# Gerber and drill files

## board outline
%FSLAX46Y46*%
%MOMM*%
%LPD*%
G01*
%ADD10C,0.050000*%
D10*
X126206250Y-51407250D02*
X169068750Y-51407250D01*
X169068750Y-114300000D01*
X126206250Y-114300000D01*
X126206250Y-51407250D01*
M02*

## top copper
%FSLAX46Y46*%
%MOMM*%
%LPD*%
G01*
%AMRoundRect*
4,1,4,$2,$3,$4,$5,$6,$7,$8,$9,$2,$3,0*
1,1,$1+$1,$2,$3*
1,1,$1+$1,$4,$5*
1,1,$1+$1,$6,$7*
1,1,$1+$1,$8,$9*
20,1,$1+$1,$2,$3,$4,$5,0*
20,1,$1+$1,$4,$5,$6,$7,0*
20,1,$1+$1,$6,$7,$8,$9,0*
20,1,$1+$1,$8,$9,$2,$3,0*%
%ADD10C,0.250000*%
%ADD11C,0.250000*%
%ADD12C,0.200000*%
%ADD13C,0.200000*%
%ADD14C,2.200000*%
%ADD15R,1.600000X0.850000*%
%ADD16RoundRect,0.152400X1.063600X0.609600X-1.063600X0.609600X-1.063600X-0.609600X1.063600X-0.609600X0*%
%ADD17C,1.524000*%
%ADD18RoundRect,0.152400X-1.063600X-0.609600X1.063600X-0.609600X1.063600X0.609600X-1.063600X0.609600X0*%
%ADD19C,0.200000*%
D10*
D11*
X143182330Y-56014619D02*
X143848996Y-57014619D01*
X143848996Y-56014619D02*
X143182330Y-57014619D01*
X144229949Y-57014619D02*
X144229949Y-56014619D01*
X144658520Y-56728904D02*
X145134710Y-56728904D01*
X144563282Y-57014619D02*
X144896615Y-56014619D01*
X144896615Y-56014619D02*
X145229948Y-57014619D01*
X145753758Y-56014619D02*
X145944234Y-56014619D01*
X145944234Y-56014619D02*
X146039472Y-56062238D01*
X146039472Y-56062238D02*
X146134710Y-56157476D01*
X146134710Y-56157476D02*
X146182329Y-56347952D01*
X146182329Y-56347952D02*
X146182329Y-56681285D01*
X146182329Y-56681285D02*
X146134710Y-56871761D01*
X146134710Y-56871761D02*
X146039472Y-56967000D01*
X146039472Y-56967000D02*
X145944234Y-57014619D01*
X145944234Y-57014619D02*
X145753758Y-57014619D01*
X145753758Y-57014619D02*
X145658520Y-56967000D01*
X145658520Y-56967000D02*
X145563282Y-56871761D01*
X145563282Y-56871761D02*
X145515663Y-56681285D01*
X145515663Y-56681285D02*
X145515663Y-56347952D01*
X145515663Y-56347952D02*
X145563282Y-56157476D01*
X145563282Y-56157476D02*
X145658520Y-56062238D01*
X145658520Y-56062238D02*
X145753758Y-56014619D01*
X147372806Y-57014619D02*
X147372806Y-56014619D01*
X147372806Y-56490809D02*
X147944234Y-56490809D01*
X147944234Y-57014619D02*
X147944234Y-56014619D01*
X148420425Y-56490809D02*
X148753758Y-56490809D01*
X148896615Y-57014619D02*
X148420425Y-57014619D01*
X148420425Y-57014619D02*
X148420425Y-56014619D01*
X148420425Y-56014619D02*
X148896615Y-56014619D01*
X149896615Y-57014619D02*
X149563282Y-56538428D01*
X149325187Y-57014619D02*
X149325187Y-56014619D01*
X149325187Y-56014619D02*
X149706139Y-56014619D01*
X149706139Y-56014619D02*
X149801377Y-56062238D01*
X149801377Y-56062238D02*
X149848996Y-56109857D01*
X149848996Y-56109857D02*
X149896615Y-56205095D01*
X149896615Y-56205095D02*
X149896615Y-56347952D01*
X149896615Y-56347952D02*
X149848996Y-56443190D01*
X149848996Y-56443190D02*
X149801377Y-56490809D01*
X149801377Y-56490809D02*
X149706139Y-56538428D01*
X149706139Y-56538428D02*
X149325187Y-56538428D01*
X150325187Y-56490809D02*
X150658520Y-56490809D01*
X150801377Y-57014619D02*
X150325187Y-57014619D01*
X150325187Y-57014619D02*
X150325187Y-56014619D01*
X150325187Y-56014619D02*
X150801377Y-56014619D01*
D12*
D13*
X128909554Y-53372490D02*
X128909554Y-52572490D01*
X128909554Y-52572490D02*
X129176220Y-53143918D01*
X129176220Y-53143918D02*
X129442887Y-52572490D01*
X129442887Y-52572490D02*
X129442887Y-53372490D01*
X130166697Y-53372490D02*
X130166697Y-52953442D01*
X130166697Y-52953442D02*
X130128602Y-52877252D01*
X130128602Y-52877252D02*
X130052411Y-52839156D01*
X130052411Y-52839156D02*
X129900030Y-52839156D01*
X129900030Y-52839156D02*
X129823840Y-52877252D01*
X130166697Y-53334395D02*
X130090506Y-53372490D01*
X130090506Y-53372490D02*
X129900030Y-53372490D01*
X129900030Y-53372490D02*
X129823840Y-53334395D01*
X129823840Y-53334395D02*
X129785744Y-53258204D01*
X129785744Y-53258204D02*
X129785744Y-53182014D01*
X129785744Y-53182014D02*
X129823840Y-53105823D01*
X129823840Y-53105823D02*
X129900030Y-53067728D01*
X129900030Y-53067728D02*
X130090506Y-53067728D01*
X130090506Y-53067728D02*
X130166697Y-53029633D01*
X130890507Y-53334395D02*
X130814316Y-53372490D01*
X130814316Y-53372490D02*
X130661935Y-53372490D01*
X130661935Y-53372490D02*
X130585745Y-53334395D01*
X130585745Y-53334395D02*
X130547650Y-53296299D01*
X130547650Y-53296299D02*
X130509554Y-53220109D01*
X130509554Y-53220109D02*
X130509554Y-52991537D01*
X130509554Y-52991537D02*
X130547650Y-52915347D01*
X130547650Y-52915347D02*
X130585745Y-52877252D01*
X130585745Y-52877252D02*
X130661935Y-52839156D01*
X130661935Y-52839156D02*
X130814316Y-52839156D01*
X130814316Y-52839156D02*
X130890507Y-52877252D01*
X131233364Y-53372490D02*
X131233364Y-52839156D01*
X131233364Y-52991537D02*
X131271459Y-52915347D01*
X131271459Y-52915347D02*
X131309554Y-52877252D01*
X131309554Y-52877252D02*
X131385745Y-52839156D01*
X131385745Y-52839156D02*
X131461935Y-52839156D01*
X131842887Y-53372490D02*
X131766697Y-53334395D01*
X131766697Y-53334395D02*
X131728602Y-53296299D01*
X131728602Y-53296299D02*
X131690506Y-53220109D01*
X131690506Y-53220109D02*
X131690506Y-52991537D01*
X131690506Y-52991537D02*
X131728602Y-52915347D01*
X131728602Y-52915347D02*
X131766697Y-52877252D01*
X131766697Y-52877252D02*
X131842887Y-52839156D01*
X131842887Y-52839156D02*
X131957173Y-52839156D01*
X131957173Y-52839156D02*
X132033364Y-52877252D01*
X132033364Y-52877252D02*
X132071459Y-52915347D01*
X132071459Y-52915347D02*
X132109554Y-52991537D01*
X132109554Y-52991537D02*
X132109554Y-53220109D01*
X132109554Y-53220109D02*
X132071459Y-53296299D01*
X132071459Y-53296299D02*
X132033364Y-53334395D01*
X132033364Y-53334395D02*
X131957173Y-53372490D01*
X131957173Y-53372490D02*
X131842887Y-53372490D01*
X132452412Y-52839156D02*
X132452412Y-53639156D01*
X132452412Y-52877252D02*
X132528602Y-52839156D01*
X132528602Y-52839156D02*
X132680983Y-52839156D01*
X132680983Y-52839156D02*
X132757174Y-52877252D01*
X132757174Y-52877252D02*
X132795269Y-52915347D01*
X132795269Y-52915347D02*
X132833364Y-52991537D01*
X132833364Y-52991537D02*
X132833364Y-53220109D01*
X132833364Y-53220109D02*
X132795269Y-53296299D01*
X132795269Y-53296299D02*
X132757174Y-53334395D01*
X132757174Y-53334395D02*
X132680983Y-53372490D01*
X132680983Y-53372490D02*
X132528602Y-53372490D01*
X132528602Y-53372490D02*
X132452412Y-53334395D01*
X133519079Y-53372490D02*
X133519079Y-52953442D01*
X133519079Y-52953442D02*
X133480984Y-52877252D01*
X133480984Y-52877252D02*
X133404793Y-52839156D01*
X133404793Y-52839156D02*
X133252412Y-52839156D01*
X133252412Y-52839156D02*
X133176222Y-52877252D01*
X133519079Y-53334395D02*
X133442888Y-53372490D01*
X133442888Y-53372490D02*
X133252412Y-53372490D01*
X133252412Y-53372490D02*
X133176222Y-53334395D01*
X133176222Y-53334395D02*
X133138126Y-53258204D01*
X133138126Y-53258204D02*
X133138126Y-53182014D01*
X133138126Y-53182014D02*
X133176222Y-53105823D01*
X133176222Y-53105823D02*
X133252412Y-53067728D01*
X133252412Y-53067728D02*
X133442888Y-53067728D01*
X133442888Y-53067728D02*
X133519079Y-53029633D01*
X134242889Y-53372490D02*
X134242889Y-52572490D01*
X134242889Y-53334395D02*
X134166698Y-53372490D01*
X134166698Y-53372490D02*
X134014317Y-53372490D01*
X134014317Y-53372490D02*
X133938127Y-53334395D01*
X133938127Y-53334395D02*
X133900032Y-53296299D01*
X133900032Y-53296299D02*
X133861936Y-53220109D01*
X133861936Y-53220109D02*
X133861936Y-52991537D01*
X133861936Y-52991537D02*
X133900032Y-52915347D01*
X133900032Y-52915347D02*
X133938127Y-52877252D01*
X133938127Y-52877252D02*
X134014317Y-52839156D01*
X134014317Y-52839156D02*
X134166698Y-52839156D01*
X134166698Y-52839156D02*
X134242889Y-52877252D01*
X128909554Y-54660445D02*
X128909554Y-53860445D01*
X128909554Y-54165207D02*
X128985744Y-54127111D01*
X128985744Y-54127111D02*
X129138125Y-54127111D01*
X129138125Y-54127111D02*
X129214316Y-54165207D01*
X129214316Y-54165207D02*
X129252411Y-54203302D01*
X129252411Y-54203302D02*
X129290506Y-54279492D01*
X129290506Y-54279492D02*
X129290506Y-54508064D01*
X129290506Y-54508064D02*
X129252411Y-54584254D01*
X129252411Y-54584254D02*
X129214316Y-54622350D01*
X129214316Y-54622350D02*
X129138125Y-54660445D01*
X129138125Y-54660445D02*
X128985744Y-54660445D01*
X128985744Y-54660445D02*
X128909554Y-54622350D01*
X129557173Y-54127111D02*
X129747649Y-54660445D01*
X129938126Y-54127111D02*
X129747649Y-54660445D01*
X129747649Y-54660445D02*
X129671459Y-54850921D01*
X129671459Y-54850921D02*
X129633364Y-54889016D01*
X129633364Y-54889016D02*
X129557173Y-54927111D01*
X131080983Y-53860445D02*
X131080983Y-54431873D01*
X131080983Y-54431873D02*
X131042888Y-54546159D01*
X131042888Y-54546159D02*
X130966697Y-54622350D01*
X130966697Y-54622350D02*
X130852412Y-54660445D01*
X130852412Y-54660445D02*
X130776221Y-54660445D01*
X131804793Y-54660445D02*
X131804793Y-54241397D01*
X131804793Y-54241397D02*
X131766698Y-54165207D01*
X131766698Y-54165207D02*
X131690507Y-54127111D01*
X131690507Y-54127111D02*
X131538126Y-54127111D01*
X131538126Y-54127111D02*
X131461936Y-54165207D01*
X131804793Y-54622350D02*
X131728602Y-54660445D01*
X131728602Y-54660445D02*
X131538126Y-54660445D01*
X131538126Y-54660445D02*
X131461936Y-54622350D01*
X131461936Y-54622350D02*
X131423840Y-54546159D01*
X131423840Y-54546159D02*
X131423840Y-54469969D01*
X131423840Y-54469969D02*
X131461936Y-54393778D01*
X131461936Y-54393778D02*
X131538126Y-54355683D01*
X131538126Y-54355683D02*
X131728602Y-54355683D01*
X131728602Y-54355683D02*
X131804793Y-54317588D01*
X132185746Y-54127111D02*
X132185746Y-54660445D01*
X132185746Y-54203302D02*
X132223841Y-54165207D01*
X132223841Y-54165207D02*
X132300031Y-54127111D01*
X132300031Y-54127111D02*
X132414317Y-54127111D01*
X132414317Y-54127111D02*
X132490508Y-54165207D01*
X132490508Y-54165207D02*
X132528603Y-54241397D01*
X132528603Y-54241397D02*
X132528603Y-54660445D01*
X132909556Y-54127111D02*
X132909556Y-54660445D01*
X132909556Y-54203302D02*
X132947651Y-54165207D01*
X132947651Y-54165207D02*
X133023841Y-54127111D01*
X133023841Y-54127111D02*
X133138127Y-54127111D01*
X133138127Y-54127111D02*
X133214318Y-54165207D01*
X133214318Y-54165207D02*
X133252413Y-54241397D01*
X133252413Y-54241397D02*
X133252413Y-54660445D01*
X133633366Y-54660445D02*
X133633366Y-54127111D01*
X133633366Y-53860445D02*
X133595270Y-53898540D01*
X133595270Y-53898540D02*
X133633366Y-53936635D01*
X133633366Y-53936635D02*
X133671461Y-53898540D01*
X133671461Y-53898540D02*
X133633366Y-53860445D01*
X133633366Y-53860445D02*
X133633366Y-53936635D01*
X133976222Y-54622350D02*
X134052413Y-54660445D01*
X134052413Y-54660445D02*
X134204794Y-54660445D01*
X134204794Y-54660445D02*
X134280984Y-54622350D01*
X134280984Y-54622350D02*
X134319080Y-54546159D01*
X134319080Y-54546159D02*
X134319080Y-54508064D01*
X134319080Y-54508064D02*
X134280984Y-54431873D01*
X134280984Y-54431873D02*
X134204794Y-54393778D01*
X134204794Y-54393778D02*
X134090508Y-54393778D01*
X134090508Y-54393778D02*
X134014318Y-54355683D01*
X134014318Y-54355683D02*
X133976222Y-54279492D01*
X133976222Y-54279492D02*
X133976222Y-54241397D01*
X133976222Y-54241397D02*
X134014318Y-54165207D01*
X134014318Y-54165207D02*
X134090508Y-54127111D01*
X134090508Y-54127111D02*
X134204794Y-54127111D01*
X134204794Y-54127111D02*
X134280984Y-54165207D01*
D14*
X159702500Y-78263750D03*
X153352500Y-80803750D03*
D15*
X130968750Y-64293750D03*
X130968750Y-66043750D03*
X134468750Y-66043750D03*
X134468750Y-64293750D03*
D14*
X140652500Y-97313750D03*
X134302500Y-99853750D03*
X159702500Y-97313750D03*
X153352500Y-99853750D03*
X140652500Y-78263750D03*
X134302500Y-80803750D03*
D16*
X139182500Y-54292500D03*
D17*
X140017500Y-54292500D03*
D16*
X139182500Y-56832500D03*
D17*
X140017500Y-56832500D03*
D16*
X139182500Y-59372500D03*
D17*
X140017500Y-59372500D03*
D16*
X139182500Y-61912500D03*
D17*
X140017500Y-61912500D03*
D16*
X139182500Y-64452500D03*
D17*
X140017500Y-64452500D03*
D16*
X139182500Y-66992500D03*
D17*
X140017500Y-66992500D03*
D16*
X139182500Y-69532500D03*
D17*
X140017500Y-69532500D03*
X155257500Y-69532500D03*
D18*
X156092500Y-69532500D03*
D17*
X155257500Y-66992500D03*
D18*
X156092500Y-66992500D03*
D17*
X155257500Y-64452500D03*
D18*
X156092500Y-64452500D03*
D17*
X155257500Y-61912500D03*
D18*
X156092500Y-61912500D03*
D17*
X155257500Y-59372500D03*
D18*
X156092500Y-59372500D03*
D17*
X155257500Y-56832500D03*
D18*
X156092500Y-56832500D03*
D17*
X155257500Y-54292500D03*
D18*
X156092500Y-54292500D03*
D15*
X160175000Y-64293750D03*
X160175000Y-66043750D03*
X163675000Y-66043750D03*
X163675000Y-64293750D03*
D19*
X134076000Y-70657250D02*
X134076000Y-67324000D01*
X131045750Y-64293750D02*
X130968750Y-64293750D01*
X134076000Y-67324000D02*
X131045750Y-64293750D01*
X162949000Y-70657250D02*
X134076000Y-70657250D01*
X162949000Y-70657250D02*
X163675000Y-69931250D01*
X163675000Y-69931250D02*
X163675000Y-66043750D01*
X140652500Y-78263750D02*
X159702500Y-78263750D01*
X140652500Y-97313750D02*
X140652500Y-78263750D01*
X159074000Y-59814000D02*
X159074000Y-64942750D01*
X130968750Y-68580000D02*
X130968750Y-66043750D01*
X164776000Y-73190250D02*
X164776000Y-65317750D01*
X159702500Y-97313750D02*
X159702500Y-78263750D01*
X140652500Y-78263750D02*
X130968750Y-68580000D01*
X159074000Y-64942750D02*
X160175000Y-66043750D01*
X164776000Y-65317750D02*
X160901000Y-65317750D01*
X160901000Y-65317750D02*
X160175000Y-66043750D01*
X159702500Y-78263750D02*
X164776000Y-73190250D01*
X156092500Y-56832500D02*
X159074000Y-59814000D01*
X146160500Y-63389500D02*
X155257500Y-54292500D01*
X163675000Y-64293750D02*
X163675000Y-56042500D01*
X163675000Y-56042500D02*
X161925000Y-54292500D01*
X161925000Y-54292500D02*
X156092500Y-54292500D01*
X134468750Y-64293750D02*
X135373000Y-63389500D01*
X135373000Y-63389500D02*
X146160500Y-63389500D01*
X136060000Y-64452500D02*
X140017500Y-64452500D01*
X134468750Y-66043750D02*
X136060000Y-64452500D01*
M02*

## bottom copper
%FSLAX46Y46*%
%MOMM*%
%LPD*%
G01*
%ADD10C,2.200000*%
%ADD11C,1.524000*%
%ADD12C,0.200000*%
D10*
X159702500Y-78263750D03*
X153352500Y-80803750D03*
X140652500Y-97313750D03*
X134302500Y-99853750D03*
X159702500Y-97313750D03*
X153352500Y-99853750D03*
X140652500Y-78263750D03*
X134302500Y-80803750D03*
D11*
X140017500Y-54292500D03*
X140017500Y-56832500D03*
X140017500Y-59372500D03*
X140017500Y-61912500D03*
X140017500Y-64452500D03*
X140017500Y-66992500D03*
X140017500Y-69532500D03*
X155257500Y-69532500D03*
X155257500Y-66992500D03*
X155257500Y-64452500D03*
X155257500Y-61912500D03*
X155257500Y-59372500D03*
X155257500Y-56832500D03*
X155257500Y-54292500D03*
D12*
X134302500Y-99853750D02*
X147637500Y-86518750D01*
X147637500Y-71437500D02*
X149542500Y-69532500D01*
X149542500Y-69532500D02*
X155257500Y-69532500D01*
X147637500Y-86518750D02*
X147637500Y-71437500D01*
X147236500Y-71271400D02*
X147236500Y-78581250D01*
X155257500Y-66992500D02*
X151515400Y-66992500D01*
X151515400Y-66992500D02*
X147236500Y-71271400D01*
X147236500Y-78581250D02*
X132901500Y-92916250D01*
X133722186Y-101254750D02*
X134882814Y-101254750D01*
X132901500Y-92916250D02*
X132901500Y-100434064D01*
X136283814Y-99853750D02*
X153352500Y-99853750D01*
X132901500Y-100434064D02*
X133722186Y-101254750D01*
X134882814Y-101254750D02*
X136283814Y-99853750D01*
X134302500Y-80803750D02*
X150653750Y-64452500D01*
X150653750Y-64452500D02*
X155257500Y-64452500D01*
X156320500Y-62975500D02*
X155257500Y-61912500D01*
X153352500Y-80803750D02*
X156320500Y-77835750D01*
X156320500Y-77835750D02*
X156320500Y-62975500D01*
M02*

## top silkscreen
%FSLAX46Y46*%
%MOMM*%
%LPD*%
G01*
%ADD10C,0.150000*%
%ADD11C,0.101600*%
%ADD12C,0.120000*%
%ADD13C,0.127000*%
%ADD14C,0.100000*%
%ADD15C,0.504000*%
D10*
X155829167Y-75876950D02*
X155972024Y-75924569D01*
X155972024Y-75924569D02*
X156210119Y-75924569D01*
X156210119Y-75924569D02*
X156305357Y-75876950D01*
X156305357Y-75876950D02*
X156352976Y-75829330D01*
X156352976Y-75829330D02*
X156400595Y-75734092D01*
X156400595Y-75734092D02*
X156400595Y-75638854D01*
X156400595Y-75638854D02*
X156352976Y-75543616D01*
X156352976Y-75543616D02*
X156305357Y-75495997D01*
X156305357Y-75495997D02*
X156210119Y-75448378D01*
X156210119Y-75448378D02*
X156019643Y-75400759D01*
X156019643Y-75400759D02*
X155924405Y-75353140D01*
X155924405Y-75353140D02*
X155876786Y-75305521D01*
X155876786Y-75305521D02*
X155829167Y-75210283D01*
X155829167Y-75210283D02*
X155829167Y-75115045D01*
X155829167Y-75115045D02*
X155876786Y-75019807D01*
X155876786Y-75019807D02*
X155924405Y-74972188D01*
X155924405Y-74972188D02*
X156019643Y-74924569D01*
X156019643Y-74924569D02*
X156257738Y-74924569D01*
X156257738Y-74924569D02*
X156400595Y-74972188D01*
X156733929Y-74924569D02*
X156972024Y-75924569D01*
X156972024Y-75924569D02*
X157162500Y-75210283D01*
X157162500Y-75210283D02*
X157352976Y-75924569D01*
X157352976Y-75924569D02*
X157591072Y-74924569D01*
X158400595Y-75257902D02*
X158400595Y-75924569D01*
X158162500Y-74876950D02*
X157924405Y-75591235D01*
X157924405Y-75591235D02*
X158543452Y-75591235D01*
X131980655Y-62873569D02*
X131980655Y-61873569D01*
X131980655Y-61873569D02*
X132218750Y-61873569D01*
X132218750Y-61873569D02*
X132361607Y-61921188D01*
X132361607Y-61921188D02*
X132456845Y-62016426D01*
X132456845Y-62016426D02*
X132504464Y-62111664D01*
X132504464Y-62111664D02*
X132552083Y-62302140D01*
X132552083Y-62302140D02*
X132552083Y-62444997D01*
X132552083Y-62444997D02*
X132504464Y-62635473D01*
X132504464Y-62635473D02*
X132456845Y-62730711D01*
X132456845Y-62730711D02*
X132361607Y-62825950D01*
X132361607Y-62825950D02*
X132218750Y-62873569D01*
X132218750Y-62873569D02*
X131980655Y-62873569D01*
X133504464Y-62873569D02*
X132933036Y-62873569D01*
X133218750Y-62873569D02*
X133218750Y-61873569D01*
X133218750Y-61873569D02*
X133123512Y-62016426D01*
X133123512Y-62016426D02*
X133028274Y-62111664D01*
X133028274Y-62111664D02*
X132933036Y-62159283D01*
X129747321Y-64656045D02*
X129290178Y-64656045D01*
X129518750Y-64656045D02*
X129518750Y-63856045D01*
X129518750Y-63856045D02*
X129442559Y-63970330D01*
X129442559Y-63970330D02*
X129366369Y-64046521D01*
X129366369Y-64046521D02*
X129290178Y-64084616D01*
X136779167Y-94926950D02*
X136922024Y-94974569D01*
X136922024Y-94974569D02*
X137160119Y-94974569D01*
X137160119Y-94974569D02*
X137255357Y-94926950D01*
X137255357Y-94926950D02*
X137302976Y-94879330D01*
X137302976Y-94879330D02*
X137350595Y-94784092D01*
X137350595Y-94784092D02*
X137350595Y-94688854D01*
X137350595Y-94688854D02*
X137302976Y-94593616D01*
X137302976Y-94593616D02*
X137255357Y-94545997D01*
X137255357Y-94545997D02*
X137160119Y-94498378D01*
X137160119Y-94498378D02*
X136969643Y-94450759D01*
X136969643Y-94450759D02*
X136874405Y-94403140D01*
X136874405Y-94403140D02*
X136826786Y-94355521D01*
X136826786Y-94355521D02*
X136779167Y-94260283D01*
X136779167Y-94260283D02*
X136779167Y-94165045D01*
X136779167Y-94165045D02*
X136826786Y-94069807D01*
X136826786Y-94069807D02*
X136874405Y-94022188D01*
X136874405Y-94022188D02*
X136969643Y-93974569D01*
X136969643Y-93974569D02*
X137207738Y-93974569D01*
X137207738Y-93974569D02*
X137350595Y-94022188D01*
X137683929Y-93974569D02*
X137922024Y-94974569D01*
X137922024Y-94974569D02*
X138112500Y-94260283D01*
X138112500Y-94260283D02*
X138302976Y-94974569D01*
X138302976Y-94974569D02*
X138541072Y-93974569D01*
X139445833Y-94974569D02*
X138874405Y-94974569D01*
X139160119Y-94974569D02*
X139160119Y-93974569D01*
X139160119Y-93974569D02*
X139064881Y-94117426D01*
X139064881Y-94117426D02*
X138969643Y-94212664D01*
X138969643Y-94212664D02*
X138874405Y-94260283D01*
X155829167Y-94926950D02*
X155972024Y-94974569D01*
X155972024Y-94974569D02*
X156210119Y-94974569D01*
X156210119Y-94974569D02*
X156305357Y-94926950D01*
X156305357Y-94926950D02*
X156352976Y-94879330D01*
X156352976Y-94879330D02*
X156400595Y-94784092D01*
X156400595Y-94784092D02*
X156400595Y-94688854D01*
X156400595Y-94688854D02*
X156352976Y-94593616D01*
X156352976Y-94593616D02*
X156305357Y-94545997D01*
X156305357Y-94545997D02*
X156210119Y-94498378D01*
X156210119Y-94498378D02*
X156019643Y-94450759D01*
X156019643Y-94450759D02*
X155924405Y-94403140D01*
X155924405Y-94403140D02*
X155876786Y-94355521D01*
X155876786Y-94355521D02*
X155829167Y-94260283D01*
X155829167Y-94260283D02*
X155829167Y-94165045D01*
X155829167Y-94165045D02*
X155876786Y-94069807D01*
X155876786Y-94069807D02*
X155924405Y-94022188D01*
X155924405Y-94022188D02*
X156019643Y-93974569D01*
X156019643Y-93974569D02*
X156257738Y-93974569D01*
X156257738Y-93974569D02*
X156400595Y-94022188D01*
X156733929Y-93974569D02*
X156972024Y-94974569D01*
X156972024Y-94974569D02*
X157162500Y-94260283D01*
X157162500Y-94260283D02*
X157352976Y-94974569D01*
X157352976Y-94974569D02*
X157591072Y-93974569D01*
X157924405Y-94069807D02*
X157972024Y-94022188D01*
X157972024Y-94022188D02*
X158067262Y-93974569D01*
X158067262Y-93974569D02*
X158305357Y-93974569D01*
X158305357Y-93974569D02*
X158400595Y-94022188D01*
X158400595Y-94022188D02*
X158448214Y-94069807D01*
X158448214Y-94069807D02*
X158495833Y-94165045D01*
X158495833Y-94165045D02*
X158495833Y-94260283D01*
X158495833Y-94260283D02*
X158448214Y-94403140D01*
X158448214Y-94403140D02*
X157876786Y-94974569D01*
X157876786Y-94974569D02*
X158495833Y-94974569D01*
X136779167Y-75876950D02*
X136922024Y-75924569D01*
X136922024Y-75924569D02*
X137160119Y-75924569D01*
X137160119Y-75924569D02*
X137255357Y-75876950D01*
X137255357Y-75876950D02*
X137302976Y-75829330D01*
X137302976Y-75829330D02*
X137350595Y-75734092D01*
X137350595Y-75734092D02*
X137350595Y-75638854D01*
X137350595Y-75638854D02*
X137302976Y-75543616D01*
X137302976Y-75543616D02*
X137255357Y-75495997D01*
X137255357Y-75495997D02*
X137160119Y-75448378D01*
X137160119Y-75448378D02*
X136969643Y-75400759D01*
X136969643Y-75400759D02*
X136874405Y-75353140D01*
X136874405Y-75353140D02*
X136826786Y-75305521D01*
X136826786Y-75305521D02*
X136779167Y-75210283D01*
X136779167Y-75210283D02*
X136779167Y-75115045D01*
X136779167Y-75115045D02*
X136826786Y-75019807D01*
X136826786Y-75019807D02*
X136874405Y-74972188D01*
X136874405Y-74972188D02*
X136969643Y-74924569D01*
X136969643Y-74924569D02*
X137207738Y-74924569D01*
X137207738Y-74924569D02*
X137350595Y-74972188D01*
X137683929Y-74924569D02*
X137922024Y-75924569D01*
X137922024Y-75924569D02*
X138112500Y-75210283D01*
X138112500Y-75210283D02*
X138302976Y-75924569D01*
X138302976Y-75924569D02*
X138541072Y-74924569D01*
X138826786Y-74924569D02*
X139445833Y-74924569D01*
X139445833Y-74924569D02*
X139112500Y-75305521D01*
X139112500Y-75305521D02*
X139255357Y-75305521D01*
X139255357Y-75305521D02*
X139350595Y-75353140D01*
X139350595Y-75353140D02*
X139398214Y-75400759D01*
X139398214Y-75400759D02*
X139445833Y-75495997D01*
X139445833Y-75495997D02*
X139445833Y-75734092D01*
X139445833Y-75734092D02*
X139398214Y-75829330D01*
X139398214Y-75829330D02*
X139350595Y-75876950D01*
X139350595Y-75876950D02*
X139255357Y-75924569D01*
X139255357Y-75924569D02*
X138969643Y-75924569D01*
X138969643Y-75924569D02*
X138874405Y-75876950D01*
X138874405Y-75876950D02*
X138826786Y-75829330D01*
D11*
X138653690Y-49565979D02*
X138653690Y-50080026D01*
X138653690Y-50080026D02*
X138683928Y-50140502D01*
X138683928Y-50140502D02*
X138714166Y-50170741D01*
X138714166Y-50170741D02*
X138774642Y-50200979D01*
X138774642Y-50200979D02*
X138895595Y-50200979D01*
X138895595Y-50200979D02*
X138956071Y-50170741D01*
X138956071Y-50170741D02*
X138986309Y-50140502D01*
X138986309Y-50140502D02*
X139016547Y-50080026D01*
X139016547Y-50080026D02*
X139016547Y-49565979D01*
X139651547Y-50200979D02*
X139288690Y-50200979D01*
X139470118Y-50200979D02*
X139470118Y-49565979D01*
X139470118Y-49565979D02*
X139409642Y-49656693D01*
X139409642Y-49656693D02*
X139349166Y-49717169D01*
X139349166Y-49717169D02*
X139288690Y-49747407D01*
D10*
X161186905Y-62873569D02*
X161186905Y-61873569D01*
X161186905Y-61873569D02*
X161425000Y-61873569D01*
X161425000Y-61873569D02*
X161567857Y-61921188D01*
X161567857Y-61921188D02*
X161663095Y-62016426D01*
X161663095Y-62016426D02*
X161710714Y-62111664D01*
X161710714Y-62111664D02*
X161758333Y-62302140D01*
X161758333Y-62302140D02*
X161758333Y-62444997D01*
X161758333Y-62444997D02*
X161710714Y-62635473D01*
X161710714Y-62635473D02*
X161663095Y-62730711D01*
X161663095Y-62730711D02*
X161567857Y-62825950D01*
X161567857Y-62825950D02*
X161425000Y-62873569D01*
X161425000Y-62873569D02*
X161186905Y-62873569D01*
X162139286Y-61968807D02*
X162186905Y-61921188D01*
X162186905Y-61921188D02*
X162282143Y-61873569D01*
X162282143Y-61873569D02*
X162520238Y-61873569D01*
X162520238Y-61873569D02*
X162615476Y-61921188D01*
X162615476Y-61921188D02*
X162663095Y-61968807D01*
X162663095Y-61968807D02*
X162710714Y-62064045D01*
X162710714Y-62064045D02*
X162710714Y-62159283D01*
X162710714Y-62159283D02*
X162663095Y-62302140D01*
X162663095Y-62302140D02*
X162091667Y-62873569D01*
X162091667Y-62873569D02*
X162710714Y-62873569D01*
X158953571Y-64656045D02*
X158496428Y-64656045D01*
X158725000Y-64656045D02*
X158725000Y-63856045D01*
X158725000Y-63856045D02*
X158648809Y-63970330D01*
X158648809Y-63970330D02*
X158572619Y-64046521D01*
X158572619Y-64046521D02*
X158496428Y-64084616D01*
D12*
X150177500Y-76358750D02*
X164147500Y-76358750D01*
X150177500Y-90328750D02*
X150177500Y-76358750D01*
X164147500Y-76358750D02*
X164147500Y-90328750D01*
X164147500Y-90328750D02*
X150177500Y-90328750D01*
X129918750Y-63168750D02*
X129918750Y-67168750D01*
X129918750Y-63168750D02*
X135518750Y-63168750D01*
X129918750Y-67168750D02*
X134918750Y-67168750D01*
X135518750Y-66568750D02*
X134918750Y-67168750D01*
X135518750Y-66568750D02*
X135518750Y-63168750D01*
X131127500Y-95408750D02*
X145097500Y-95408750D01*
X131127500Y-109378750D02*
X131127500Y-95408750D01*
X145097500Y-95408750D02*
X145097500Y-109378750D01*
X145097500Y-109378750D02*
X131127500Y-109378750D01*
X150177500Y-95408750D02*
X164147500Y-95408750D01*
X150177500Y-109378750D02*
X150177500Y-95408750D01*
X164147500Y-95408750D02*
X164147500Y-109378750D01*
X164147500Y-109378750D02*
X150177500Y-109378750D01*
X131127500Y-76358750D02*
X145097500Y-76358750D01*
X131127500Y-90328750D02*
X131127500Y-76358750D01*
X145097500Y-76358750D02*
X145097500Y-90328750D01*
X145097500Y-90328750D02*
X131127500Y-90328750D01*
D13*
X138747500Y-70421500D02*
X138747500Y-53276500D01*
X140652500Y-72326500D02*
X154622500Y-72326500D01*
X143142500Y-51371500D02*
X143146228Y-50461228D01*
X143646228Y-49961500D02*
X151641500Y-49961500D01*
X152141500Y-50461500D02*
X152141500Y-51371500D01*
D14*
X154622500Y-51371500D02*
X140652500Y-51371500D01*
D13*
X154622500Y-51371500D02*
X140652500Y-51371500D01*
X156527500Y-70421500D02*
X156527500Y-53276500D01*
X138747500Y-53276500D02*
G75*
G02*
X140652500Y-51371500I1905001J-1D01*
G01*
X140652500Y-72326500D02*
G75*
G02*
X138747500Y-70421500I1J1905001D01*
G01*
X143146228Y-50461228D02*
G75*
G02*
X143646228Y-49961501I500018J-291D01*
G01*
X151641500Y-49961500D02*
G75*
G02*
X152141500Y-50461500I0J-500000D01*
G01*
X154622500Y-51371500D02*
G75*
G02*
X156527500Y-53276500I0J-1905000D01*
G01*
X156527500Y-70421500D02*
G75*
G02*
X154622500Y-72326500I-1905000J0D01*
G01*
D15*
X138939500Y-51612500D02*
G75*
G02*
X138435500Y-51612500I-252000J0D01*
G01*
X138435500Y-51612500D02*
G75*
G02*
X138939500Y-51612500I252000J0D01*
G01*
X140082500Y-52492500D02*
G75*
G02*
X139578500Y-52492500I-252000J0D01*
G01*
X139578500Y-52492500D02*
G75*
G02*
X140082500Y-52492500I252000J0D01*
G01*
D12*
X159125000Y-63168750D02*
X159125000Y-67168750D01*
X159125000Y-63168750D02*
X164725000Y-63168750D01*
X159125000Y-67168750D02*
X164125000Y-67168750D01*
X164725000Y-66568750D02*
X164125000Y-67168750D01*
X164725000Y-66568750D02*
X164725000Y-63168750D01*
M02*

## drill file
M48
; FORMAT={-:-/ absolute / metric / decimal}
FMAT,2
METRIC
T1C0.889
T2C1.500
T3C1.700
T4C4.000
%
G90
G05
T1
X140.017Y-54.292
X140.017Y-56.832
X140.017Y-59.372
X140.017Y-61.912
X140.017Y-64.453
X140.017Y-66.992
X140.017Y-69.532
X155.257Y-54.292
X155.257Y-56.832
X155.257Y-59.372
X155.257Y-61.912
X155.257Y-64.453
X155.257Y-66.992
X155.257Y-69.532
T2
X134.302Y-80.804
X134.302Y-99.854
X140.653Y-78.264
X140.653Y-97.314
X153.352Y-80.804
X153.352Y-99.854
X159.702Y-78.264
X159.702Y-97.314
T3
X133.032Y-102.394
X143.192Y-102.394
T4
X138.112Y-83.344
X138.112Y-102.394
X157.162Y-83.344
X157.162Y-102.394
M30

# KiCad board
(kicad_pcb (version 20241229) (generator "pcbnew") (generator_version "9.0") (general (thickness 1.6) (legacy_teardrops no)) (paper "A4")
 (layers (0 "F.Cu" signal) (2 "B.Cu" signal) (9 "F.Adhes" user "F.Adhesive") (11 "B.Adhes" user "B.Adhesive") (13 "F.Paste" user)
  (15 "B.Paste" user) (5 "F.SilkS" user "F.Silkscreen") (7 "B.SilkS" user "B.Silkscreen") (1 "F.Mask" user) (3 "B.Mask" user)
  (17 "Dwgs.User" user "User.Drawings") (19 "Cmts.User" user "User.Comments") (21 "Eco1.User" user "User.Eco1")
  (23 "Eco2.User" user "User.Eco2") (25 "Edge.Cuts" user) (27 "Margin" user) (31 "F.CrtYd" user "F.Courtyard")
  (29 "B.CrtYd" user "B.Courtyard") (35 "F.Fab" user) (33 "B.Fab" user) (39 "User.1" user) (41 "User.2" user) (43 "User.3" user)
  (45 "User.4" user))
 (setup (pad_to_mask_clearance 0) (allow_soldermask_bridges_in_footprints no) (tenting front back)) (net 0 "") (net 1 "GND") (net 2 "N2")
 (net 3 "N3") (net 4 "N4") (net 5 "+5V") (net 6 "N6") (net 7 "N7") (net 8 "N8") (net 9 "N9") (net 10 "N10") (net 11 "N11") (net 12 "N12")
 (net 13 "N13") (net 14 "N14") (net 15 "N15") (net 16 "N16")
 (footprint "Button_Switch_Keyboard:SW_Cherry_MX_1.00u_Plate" (layer "F.Cu") (at 159.7025 78.26375)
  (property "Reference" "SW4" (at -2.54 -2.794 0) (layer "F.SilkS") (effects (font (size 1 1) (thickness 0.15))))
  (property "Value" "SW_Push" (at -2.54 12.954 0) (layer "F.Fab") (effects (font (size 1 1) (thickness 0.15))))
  (fp_line (start -9.525 -1.905) (end 4.445 -1.905) (stroke (width 0.12) (type solid)) (layer "F.SilkS"))
  (fp_line (start -9.525 12.065) (end -9.525 -1.905) (stroke (width 0.12) (type solid)) (layer "F.SilkS"))
  (fp_line (start 4.445 -1.905) (end 4.445 12.065) (stroke (width 0.12) (type solid)) (layer "F.SilkS"))
  (fp_line (start 4.445 12.065) (end -9.525 12.065) (stroke (width 0.12) (type solid)) (layer "F.SilkS"))
  (pad "" np_thru_hole circle (at -2.54 5.08) (size 4 4) (drill 4) (layers "*.Cu" "*.Mask"))
  (pad "1" thru_hole circle (at 0 0) (size 2.2 2.2) (drill 1.5) (layers "*.Cu" "*.Mask") (remove_unused_layers no) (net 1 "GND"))
  (pad "2" thru_hole circle (at -6.35 2.54) (size 2.2 2.2) (drill 1.5) (layers "*.Cu" "*.Mask") (remove_unused_layers no) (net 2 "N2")))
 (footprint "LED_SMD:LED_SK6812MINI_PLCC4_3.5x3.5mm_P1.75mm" (layer "F.Cu") (at 132.71875 65.16875)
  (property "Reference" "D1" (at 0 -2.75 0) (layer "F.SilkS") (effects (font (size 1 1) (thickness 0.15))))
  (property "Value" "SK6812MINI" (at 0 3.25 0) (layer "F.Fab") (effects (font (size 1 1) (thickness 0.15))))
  (fp_line (start -2.8 -2) (end -2.8 2) (stroke (width 0.12) (type default)) (layer "F.SilkS"))
  (fp_line (start -2.8 -2) (end 2.8 -2) (stroke (width 0.12) (type solid)) (layer "F.SilkS"))
  (fp_line (start -2.8 2) (end 2.2 2) (stroke (width 0.12) (type solid)) (layer "F.SilkS"))
  (fp_line (start 2.8 1.4) (end 2.2 2) (stroke (width 0.12) (type default)) (layer "F.SilkS"))
  (fp_line (start 2.8 1.4) (end 2.8 -2) (stroke (width 0.12) (type solid)) (layer "F.SilkS"))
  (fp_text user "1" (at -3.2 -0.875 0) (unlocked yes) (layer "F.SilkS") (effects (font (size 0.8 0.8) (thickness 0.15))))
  (pad "1" smd rect (at -1.75 -0.875) (size 1.6 0.85) (layers "F.Cu" "F.Mask" "F.Paste") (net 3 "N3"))
  (pad "2" smd rect (at -1.75 0.875) (size 1.6 0.85) (layers "F.Cu" "F.Mask" "F.Paste") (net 1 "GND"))
  (pad "3" smd rect (at 1.75 0.875) (size 1.6 0.85) (layers "F.Cu" "F.Mask" "F.Paste") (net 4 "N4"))
  (pad "4" smd rect (at 1.75 -0.875) (size 1.6 0.85) (layers "F.Cu" "F.Mask" "F.Paste") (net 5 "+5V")))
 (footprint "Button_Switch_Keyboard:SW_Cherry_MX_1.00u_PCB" (layer "F.Cu") (at 140.6525 97.31375)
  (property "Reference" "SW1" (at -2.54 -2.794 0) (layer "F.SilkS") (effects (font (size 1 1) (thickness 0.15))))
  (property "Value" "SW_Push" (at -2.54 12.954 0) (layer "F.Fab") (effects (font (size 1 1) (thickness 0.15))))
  (fp_line (start -9.525 -1.905) (end 4.445 -1.905) (stroke (width 0.12) (type solid)) (layer "F.SilkS"))
  (fp_line (start -9.525 12.065) (end -9.525 -1.905) (stroke (width 0.12) (type solid)) (layer "F.SilkS"))
  (fp_line (start 4.445 -1.905) (end 4.445 12.065) (stroke (width 0.12) (type solid)) (layer "F.SilkS"))
  (fp_line (start 4.445 12.065) (end -9.525 12.065) (stroke (width 0.12) (type solid)) (layer "F.SilkS"))
  (pad "" np_thru_hole circle (at -7.62 5.08) (size 1.7 1.7) (drill 1.7) (layers "*.Cu" "*.Mask"))
  (pad "" np_thru_hole circle (at -2.54 5.08) (size 4 4) (drill 4) (layers "*.Cu" "*.Mask"))
  (pad "" np_thru_hole circle (at 2.54 5.08) (size 1.7 1.7) (drill 1.7) (layers "*.Cu" "*.Mask"))
  (pad "1" thru_hole circle (at 0 0) (size 2.2 2.2) (drill 1.5) (layers "*.Cu" "*.Mask") (remove_unused_layers no) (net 1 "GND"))
  (pad "2" thru_hole circle (at -6.35 2.54) (size 2.2 2.2) (drill 1.5) (layers "*.Cu" "*.Mask") (remove_unused_layers no) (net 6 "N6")))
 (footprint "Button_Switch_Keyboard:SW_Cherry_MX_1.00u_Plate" (layer "F.Cu") (at 159.7025 97.31375)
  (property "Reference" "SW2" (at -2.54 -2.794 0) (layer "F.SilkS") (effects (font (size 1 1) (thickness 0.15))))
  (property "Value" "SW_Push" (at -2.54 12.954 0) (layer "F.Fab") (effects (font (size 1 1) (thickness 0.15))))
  (fp_line (start -9.525 -1.905) (end 4.445 -1.905) (stroke (width 0.12) (type solid)) (layer "F.SilkS"))
  (fp_line (start -9.525 12.065) (end -9.525 -1.905) (stroke (width 0.12) (type solid)) (layer "F.SilkS"))
  (fp_line (start 4.445 -1.905) (end 4.445 12.065) (stroke (width 0.12) (type solid)) (layer "F.SilkS"))
  (fp_line (start 4.445 12.065) (end -9.525 12.065) (stroke (width 0.12) (type solid)) (layer "F.SilkS"))
  (pad "" np_thru_hole circle (at -2.54 5.08) (size 4 4) (drill 4) (layers "*.Cu" "*.Mask"))
  (pad "1" thru_hole circle (at 0 0) (size 2.2 2.2) (drill 1.5) (layers "*.Cu" "*.Mask") (remove_unused_layers no) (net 1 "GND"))
  (pad "2" thru_hole circle (at -6.35 2.54) (size 2.2 2.2) (drill 1.5) (layers "*.Cu" "*.Mask") (remove_unused_layers no) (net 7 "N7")))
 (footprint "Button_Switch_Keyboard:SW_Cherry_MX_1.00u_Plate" (layer "F.Cu") (at 140.6525 78.26375)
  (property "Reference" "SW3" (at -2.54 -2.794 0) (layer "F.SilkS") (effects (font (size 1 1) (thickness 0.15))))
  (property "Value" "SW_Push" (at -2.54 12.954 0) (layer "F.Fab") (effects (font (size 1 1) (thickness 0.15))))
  (fp_line (start -9.525 -1.905) (end 4.445 -1.905) (stroke (width 0.12) (type solid)) (layer "F.SilkS"))
  (fp_line (start -9.525 12.065) (end -9.525 -1.905) (stroke (width 0.12) (type solid)) (layer "F.SilkS"))
  (fp_line (start 4.445 -1.905) (end 4.445 12.065) (stroke (width 0.12) (type solid)) (layer "F.SilkS"))
  (fp_line (start 4.445 12.065) (end -9.525 12.065) (stroke (width 0.12) (type solid)) (layer "F.SilkS"))
  (pad "" np_thru_hole circle (at -2.54 5.08) (size 4 4) (drill 4) (layers "*.Cu" "*.Mask"))
  (pad "1" thru_hole circle (at 0 0) (size 2.2 2.2) (drill 1.5) (layers "*.Cu" "*.Mask") (remove_unused_layers no) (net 1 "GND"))
  (pad "2" thru_hole circle (at -6.35 2.54) (size 2.2 2.2) (drill 1.5) (layers "*.Cu" "*.Mask") (remove_unused_layers no) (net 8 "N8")))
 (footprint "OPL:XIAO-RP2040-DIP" (layer "F.Cu") (at 147.6375 61.9125)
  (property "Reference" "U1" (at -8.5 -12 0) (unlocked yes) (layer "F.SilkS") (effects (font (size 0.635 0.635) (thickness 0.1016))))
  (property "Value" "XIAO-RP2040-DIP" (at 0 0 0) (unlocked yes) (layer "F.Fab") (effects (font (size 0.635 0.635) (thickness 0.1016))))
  (fp_line (start -8.89 8.509) (end -8.89 -8.636) (stroke (width 0.127) (type solid)) (layer "F.SilkS"))
  (fp_line (start -6.985 10.414) (end 6.985 10.414) (stroke (width 0.127) (type solid)) (layer "F.SilkS"))
  (fp_line (start -4.495 -10.541) (end -4.491272 -11.451272) (stroke (width 0.127) (type solid)) (layer "F.SilkS"))
  (fp_line (start -3.991272 -11.951) (end 4.004 -11.951) (stroke (width 0.127) (type solid)) (layer "F.SilkS"))
  (fp_line (start 4.504 -11.451) (end 4.504 -10.541) (stroke (width 0.127) (type solid)) (layer "F.SilkS"))
  (fp_line (start 6.985 -10.541) (end -6.985 -10.541) (stroke (width 0.1) (type solid)) (layer "F.SilkS"))
  (fp_line (start 6.985 -10.541) (end -6.985 -10.541) (stroke (width 0.127) (type solid)) (layer "F.SilkS"))
  (fp_line (start 8.89 8.509) (end 8.89 -8.636) (stroke (width 0.127) (type solid)) (layer "F.SilkS"))
  (fp_arc (start -8.89 -8.636) (mid -8.332038 -9.983038) (end -6.985 -10.541) (stroke (width 0.127) (type solid)) (layer "F.SilkS"))
  (fp_arc (start -6.985 10.414) (mid -8.332038 9.856038) (end -8.89 8.509) (stroke (width 0.127) (type solid)) (layer "F.SilkS"))
  (fp_arc (start -4.491272 -11.451272) (mid -4.344728 -11.80464) (end -3.991272 -11.951) (stroke (width 0.127) (type default))
   (layer "F.SilkS"))
  (fp_arc (start 4.004 -11.951) (mid 4.357553 -11.804553) (end 4.504 -11.451) (stroke (width 0.127) (type default)) (layer "F.SilkS"))
  (fp_arc (start 6.985 -10.541) (mid 8.332038 -9.983038) (end 8.89 -8.636) (stroke (width 0.127) (type solid)) (layer "F.SilkS"))
  (fp_arc (start 8.89 8.509) (mid 8.332038 9.856038) (end 6.985 10.414) (stroke (width 0.127) (type solid)) (layer "F.SilkS"))
  (fp_circle (center -8.95 -10.3) (end -8.95 -10.554) (stroke (width 0.5) (type solid)) (fill yes) (layer "F.SilkS"))
  (fp_circle (center -7.807 -9.42) (end -7.807 -9.674) (stroke (width 0.5) (type solid)) (fill yes) (layer "F.SilkS"))
  (pad "1" smd roundrect (at -8.455 -7.62 180) (size 2.432 1.524) (layers "F.Cu" "F.Mask") (roundrect_rratio 0.1) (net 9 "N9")
   (thermal_bridge_angle 45))
  (pad "1" thru_hole circle (at -7.62 -7.62 180) (size 1.524 1.524) (drill 0.889) (layers "*.Cu" "*.Mask") (remove_unused_layers no)
   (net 9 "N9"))
  (pad "2" smd roundrect (at -8.455 -5.08 180) (size 2.432 1.524) (layers "F.Cu" "F.Mask") (roundrect_rratio 0.1) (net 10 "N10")
   (thermal_bridge_angle 45))
  (pad "2" thru_hole circle (at -7.62 -5.08 180) (size 1.524 1.524) (drill 0.889) (layers "*.Cu" "*.Mask") (remove_unused_layers no)
   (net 10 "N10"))
  (pad "3" smd roundrect (at -8.455 -2.54 180) (size 2.432 1.524) (layers "F.Cu" "F.Mask") (roundrect_rratio 0.1) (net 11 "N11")
   (thermal_bridge_angle 45))
  (pad "3" thru_hole circle (at -7.62 -2.54 180) (size 1.524 1.524) (drill 0.889) (layers "*.Cu" "*.Mask") (remove_unused_layers no)
   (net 11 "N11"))
  (pad "4" smd roundrect (at -8.455 0 180) (size 2.432 1.524) (layers "F.Cu" "F.Mask") (roundrect_rratio 0.1) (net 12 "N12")
   (thermal_bridge_angle 45))
  (pad "4" thru_hole circle (at -7.62 0 180) (size 1.524 1.524) (drill 0.889) (layers "*.Cu" "*.Mask") (remove_unused_layers no)
   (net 12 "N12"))
  (pad "5" smd roundrect (at -8.455 2.54 180) (size 2.432 1.524) (layers "F.Cu" "F.Mask") (roundrect_rratio 0.1) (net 4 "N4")
   (thermal_bridge_angle 45))
  (pad "5" thru_hole circle (at -7.62 2.54 180) (size 1.524 1.524) (drill 0.889) (layers "*.Cu" "*.Mask") (remove_unused_layers no)
   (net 4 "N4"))
  (pad "6" smd roundrect (at -8.455 5.08 180) (size 2.432 1.524) (layers "F.Cu" "F.Mask") (roundrect_rratio 0.1) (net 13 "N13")
   (thermal_bridge_angle 45))
  (pad "6" thru_hole circle (at -7.62 5.08 180) (size 1.524 1.524) (drill 0.889) (layers "*.Cu" "*.Mask") (remove_unused_layers no)
   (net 13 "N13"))
  (pad "7" smd roundrect (at -8.455 7.62 180) (size 2.432 1.524) (layers "F.Cu" "F.Mask") (roundrect_rratio 0.1) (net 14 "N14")
   (thermal_bridge_angle 45))
  (pad "7" thru_hole circle (at -7.62 7.62 180) (size 1.524 1.524) (drill 0.889) (layers "*.Cu" "*.Mask") (remove_unused_layers no)
   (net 14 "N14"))
  (pad "8" thru_hole circle (at 7.62 7.62) (size 1.524 1.524) (drill 0.889) (layers "*.Cu" "*.Mask") (remove_unused_layers no) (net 6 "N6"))
  (pad "8" smd roundrect (at 8.455 7.62) (size 2.432 1.524) (layers "F.Cu" "F.Mask") (roundrect_rratio 0.1) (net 6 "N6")
   (thermal_bridge_angle 45))
  (pad "9" thru_hole circle (at 7.62 5.08) (size 1.524 1.524) (drill 0.889) (layers "*.Cu" "*.Mask") (remove_unused_layers no) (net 7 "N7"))
  (pad "9" smd roundrect (at 8.455 5.08) (size 2.432 1.524) (layers "F.Cu" "F.Mask") (roundrect_rratio 0.1) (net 7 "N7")
   (thermal_bridge_angle 45))
  (pad "10" thru_hole circle (at 7.62 2.54) (size 1.524 1.524) (drill 0.889) (layers "*.Cu" "*.Mask") (remove_unused_layers no) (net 8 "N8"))
  (pad "10" smd roundrect (at 8.455 2.54) (size 2.432 1.524) (layers "F.Cu" "F.Mask") (roundrect_rratio 0.1) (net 8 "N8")
   (thermal_bridge_angle 45))
  (pad "11" thru_hole circle (at 7.62 0) (size 1.524 1.524) (drill 0.889) (layers "*.Cu" "*.Mask") (remove_unused_layers no) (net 2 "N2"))
  (pad "11" smd roundrect (at 8.455 0) (size 2.432 1.524) (layers "F.Cu" "F.Mask") (roundrect_rratio 0.1) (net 2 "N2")
   (thermal_bridge_angle 45))
  (pad "12" thru_hole circle (at 7.62 -2.54) (size 1.524 1.524) (drill 0.889) (layers "*.Cu" "*.Mask") (remove_unused_layers no)
   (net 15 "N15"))
  (pad "12" smd roundrect (at 8.455 -2.54) (size 2.432 1.524) (layers "F.Cu" "F.Mask") (roundrect_rratio 0.1) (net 15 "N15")
   (thermal_bridge_angle 45))
  (pad "13" thru_hole circle (at 7.62 -5.08) (size 1.524 1.524) (drill 0.889) (layers "*.Cu" "*.Mask") (remove_unused_layers no)
   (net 1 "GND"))
  (pad "13" smd roundrect (at 8.455 -5.08) (size 2.432 1.524) (layers "F.Cu" "F.Mask") (roundrect_rratio 0.1) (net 1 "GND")
   (thermal_bridge_angle 45))
  (pad "14" thru_hole circle (at 7.62 -7.62) (size 1.524 1.524) (drill 0.889) (layers "*.Cu" "*.Mask") (remove_unused_layers no)
   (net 5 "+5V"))
  (pad "14" smd roundrect (at 8.455 -7.62) (size 2.432 1.524) (layers "F.Cu" "F.Mask") (roundrect_rratio 0.1) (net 5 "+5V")
   (thermal_bridge_angle 45)))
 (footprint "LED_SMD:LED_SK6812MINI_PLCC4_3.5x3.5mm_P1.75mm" (layer "F.Cu") (at 161.925 65.16875)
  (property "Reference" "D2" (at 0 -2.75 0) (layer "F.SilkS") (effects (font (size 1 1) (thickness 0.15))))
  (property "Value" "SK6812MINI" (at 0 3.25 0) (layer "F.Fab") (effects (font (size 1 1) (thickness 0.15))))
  (fp_line (start -2.8 -2) (end -2.8 2) (stroke (width 0.12) (type default)) (layer "F.SilkS"))
  (fp_line (start -2.8 -2) (end 2.8 -2) (stroke (width 0.12) (type solid)) (layer "F.SilkS"))
  (fp_line (start -2.8 2) (end 2.2 2) (stroke (width 0.12) (type solid)) (layer "F.SilkS"))
  (fp_line (start 2.8 1.4) (end 2.2 2) (stroke (width 0.12) (type default)) (layer "F.SilkS"))
  (fp_line (start 2.8 1.4) (end 2.8 -2) (stroke (width 0.12) (type solid)) (layer "F.SilkS"))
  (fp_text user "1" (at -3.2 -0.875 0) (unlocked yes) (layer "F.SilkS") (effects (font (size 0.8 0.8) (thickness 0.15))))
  (pad "1" smd rect (at -1.75 -0.875) (size 1.6 0.85) (layers "F.Cu" "F.Mask" "F.Paste") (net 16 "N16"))
  (pad "2" smd rect (at -1.75 0.875) (size 1.6 0.85) (layers "F.Cu" "F.Mask" "F.Paste") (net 1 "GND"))
  (pad "3" smd rect (at 1.75 0.875) (size 1.6 0.85) (layers "F.Cu" "F.Mask" "F.Paste") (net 3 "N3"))
  (pad "4" smd rect (at 1.75 -0.875) (size 1.6 0.85) (layers "F.Cu" "F.Mask" "F.Paste") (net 5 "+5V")))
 (gr_rect (start 126.20625 51.40725) (end 169.06875 114.3) (stroke (width 0.05) (type default)) (fill no) (layer "Edge.Cuts"))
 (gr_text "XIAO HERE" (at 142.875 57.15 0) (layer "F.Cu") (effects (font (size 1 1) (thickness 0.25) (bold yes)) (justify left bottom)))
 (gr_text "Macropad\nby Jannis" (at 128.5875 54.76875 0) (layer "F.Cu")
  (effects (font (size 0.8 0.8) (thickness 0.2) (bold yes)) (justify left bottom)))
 (segment (start 134.076 70.65725) (end 134.076 67.324) (width 0.2) (layer "F.Cu") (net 3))
 (segment (start 131.04575 64.29375) (end 130.96875 64.29375) (width 0.2) (layer "F.Cu") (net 3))
 (segment (start 134.076 67.324) (end 131.04575 64.29375) (width 0.2) (layer "F.Cu") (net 3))
 (segment (start 162.949 70.65725) (end 134.076 70.65725) (width 0.2) (layer "F.Cu") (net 3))
 (segment (start 162.949 70.65725) (end 163.675 69.93125) (width 0.2) (layer "F.Cu") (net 3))
 (segment (start 163.675 69.93125) (end 163.675 66.04375) (width 0.2) (layer "F.Cu") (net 3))
 (segment (start 140.6525 78.26375) (end 159.7025 78.26375) (width 0.2) (layer "F.Cu") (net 1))
 (segment (start 140.6525 97.31375) (end 140.6525 78.26375) (width 0.2) (layer "F.Cu") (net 1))
 (segment (start 159.074 59.814) (end 159.074 64.94275) (width 0.2) (layer "F.Cu") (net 1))
 (segment (start 130.96875 68.58) (end 130.96875 66.04375) (width 0.2) (layer "F.Cu") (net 1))
 (segment (start 164.776 73.19025) (end 164.776 65.31775) (width 0.2) (layer "F.Cu") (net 1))
 (segment (start 159.7025 97.31375) (end 159.7025 78.26375) (width 0.2) (layer "F.Cu") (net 1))
 (segment (start 140.6525 78.26375) (end 130.96875 68.58) (width 0.2) (layer "F.Cu") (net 1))
 (segment (start 159.074 64.94275) (end 160.175 66.04375) (width 0.2) (layer "F.Cu") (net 1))
 (segment (start 164.776 65.31775) (end 160.901 65.31775) (width 0.2) (layer "F.Cu") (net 1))
 (segment (start 160.901 65.31775) (end 160.175 66.04375) (width 0.2) (layer "F.Cu") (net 1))
 (segment (start 159.7025 78.26375) (end 164.776 73.19025) (width 0.2) (layer "F.Cu") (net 1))
 (segment (start 156.0925 56.8325) (end 159.074 59.814) (width 0.2) (layer "F.Cu") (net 1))
 (segment (start 146.1605 63.3895) (end 155.2575 54.2925) (width 0.2) (layer "F.Cu") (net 5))
 (segment (start 163.675 64.29375) (end 163.675 56.0425) (width 0.2) (layer "F.Cu") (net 5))
 (segment (start 163.675 56.0425) (end 161.925 54.2925) (width 0.2) (layer "F.Cu") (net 5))
 (segment (start 161.925 54.2925) (end 156.0925 54.2925) (width 0.2) (layer "F.Cu") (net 5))
 (segment (start 134.46875 64.29375) (end 135.373 63.3895) (width 0.2) (layer "F.Cu") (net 5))
 (segment (start 135.373 63.3895) (end 146.1605 63.3895) (width 0.2) (layer "F.Cu") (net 5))
 (segment (start 136.06 64.4525) (end 140.0175 64.4525) (width 0.2) (layer "F.Cu") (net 4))
 (segment (start 134.46875 66.04375) (end 136.06 64.4525) (width 0.2) (layer "F.Cu") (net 4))
 (segment (start 134.3025 99.85375) (end 147.6375 86.51875) (width 0.2) (layer "B.Cu") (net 6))
 (segment (start 147.6375 71.4375) (end 149.5425 69.5325) (width 0.2) (layer "B.Cu") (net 6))
 (segment (start 149.5425 69.5325) (end 155.2575 69.5325) (width 0.2) (layer "B.Cu") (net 6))
 (segment (start 147.6375 86.51875) (end 147.6375 71.4375) (width 0.2) (layer "B.Cu") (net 6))
 (segment (start 147.2365 71.2714) (end 147.2365 78.58125) (width 0.2) (layer "B.Cu") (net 7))
 (segment (start 155.2575 66.9925) (end 151.5154 66.9925) (width 0.2) (layer "B.Cu") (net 7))
 (segment (start 151.5154 66.9925) (end 147.2365 71.2714) (width 0.2) (layer "B.Cu") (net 7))
 (segment (start 147.2365 78.58125) (end 132.9015 92.91625) (width 0.2) (layer "B.Cu") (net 7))
 (segment (start 133.722186 101.25475) (end 134.882814 101.25475) (width 0.2) (layer "B.Cu") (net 7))
 (segment (start 132.9015 92.91625) (end 132.9015 100.434064) (width 0.2) (layer "B.Cu") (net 7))
 (segment (start 136.283814 99.85375) (end 153.3525 99.85375) (width 0.2) (layer "B.Cu") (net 7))
 (segment (start 132.9015 100.434064) (end 133.722186 101.25475) (width 0.2) (layer "B.Cu") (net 7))
 (segment (start 134.882814 101.25475) (end 136.283814 99.85375) (width 0.2) (layer "B.Cu") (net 7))
 (segment (start 134.3025 80.80375) (end 150.65375 64.4525) (width 0.2) (layer "B.Cu") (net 8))
 (segment (start 150.65375 64.4525) (end 155.2575 64.4525) (width 0.2) (layer "B.Cu") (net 8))
 (segment (start 156.3205 62.9755) (end 155.2575 61.9125) (width 0.2) (layer "B.Cu") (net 2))
 (segment (start 153.3525 80.80375) (end 156.3205 77.83575) (width 0.2) (layer "B.Cu") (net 2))
 (segment (start 156.3205 77.83575) (end 156.3205 62.9755) (width 0.2) (layer "B.Cu") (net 2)))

